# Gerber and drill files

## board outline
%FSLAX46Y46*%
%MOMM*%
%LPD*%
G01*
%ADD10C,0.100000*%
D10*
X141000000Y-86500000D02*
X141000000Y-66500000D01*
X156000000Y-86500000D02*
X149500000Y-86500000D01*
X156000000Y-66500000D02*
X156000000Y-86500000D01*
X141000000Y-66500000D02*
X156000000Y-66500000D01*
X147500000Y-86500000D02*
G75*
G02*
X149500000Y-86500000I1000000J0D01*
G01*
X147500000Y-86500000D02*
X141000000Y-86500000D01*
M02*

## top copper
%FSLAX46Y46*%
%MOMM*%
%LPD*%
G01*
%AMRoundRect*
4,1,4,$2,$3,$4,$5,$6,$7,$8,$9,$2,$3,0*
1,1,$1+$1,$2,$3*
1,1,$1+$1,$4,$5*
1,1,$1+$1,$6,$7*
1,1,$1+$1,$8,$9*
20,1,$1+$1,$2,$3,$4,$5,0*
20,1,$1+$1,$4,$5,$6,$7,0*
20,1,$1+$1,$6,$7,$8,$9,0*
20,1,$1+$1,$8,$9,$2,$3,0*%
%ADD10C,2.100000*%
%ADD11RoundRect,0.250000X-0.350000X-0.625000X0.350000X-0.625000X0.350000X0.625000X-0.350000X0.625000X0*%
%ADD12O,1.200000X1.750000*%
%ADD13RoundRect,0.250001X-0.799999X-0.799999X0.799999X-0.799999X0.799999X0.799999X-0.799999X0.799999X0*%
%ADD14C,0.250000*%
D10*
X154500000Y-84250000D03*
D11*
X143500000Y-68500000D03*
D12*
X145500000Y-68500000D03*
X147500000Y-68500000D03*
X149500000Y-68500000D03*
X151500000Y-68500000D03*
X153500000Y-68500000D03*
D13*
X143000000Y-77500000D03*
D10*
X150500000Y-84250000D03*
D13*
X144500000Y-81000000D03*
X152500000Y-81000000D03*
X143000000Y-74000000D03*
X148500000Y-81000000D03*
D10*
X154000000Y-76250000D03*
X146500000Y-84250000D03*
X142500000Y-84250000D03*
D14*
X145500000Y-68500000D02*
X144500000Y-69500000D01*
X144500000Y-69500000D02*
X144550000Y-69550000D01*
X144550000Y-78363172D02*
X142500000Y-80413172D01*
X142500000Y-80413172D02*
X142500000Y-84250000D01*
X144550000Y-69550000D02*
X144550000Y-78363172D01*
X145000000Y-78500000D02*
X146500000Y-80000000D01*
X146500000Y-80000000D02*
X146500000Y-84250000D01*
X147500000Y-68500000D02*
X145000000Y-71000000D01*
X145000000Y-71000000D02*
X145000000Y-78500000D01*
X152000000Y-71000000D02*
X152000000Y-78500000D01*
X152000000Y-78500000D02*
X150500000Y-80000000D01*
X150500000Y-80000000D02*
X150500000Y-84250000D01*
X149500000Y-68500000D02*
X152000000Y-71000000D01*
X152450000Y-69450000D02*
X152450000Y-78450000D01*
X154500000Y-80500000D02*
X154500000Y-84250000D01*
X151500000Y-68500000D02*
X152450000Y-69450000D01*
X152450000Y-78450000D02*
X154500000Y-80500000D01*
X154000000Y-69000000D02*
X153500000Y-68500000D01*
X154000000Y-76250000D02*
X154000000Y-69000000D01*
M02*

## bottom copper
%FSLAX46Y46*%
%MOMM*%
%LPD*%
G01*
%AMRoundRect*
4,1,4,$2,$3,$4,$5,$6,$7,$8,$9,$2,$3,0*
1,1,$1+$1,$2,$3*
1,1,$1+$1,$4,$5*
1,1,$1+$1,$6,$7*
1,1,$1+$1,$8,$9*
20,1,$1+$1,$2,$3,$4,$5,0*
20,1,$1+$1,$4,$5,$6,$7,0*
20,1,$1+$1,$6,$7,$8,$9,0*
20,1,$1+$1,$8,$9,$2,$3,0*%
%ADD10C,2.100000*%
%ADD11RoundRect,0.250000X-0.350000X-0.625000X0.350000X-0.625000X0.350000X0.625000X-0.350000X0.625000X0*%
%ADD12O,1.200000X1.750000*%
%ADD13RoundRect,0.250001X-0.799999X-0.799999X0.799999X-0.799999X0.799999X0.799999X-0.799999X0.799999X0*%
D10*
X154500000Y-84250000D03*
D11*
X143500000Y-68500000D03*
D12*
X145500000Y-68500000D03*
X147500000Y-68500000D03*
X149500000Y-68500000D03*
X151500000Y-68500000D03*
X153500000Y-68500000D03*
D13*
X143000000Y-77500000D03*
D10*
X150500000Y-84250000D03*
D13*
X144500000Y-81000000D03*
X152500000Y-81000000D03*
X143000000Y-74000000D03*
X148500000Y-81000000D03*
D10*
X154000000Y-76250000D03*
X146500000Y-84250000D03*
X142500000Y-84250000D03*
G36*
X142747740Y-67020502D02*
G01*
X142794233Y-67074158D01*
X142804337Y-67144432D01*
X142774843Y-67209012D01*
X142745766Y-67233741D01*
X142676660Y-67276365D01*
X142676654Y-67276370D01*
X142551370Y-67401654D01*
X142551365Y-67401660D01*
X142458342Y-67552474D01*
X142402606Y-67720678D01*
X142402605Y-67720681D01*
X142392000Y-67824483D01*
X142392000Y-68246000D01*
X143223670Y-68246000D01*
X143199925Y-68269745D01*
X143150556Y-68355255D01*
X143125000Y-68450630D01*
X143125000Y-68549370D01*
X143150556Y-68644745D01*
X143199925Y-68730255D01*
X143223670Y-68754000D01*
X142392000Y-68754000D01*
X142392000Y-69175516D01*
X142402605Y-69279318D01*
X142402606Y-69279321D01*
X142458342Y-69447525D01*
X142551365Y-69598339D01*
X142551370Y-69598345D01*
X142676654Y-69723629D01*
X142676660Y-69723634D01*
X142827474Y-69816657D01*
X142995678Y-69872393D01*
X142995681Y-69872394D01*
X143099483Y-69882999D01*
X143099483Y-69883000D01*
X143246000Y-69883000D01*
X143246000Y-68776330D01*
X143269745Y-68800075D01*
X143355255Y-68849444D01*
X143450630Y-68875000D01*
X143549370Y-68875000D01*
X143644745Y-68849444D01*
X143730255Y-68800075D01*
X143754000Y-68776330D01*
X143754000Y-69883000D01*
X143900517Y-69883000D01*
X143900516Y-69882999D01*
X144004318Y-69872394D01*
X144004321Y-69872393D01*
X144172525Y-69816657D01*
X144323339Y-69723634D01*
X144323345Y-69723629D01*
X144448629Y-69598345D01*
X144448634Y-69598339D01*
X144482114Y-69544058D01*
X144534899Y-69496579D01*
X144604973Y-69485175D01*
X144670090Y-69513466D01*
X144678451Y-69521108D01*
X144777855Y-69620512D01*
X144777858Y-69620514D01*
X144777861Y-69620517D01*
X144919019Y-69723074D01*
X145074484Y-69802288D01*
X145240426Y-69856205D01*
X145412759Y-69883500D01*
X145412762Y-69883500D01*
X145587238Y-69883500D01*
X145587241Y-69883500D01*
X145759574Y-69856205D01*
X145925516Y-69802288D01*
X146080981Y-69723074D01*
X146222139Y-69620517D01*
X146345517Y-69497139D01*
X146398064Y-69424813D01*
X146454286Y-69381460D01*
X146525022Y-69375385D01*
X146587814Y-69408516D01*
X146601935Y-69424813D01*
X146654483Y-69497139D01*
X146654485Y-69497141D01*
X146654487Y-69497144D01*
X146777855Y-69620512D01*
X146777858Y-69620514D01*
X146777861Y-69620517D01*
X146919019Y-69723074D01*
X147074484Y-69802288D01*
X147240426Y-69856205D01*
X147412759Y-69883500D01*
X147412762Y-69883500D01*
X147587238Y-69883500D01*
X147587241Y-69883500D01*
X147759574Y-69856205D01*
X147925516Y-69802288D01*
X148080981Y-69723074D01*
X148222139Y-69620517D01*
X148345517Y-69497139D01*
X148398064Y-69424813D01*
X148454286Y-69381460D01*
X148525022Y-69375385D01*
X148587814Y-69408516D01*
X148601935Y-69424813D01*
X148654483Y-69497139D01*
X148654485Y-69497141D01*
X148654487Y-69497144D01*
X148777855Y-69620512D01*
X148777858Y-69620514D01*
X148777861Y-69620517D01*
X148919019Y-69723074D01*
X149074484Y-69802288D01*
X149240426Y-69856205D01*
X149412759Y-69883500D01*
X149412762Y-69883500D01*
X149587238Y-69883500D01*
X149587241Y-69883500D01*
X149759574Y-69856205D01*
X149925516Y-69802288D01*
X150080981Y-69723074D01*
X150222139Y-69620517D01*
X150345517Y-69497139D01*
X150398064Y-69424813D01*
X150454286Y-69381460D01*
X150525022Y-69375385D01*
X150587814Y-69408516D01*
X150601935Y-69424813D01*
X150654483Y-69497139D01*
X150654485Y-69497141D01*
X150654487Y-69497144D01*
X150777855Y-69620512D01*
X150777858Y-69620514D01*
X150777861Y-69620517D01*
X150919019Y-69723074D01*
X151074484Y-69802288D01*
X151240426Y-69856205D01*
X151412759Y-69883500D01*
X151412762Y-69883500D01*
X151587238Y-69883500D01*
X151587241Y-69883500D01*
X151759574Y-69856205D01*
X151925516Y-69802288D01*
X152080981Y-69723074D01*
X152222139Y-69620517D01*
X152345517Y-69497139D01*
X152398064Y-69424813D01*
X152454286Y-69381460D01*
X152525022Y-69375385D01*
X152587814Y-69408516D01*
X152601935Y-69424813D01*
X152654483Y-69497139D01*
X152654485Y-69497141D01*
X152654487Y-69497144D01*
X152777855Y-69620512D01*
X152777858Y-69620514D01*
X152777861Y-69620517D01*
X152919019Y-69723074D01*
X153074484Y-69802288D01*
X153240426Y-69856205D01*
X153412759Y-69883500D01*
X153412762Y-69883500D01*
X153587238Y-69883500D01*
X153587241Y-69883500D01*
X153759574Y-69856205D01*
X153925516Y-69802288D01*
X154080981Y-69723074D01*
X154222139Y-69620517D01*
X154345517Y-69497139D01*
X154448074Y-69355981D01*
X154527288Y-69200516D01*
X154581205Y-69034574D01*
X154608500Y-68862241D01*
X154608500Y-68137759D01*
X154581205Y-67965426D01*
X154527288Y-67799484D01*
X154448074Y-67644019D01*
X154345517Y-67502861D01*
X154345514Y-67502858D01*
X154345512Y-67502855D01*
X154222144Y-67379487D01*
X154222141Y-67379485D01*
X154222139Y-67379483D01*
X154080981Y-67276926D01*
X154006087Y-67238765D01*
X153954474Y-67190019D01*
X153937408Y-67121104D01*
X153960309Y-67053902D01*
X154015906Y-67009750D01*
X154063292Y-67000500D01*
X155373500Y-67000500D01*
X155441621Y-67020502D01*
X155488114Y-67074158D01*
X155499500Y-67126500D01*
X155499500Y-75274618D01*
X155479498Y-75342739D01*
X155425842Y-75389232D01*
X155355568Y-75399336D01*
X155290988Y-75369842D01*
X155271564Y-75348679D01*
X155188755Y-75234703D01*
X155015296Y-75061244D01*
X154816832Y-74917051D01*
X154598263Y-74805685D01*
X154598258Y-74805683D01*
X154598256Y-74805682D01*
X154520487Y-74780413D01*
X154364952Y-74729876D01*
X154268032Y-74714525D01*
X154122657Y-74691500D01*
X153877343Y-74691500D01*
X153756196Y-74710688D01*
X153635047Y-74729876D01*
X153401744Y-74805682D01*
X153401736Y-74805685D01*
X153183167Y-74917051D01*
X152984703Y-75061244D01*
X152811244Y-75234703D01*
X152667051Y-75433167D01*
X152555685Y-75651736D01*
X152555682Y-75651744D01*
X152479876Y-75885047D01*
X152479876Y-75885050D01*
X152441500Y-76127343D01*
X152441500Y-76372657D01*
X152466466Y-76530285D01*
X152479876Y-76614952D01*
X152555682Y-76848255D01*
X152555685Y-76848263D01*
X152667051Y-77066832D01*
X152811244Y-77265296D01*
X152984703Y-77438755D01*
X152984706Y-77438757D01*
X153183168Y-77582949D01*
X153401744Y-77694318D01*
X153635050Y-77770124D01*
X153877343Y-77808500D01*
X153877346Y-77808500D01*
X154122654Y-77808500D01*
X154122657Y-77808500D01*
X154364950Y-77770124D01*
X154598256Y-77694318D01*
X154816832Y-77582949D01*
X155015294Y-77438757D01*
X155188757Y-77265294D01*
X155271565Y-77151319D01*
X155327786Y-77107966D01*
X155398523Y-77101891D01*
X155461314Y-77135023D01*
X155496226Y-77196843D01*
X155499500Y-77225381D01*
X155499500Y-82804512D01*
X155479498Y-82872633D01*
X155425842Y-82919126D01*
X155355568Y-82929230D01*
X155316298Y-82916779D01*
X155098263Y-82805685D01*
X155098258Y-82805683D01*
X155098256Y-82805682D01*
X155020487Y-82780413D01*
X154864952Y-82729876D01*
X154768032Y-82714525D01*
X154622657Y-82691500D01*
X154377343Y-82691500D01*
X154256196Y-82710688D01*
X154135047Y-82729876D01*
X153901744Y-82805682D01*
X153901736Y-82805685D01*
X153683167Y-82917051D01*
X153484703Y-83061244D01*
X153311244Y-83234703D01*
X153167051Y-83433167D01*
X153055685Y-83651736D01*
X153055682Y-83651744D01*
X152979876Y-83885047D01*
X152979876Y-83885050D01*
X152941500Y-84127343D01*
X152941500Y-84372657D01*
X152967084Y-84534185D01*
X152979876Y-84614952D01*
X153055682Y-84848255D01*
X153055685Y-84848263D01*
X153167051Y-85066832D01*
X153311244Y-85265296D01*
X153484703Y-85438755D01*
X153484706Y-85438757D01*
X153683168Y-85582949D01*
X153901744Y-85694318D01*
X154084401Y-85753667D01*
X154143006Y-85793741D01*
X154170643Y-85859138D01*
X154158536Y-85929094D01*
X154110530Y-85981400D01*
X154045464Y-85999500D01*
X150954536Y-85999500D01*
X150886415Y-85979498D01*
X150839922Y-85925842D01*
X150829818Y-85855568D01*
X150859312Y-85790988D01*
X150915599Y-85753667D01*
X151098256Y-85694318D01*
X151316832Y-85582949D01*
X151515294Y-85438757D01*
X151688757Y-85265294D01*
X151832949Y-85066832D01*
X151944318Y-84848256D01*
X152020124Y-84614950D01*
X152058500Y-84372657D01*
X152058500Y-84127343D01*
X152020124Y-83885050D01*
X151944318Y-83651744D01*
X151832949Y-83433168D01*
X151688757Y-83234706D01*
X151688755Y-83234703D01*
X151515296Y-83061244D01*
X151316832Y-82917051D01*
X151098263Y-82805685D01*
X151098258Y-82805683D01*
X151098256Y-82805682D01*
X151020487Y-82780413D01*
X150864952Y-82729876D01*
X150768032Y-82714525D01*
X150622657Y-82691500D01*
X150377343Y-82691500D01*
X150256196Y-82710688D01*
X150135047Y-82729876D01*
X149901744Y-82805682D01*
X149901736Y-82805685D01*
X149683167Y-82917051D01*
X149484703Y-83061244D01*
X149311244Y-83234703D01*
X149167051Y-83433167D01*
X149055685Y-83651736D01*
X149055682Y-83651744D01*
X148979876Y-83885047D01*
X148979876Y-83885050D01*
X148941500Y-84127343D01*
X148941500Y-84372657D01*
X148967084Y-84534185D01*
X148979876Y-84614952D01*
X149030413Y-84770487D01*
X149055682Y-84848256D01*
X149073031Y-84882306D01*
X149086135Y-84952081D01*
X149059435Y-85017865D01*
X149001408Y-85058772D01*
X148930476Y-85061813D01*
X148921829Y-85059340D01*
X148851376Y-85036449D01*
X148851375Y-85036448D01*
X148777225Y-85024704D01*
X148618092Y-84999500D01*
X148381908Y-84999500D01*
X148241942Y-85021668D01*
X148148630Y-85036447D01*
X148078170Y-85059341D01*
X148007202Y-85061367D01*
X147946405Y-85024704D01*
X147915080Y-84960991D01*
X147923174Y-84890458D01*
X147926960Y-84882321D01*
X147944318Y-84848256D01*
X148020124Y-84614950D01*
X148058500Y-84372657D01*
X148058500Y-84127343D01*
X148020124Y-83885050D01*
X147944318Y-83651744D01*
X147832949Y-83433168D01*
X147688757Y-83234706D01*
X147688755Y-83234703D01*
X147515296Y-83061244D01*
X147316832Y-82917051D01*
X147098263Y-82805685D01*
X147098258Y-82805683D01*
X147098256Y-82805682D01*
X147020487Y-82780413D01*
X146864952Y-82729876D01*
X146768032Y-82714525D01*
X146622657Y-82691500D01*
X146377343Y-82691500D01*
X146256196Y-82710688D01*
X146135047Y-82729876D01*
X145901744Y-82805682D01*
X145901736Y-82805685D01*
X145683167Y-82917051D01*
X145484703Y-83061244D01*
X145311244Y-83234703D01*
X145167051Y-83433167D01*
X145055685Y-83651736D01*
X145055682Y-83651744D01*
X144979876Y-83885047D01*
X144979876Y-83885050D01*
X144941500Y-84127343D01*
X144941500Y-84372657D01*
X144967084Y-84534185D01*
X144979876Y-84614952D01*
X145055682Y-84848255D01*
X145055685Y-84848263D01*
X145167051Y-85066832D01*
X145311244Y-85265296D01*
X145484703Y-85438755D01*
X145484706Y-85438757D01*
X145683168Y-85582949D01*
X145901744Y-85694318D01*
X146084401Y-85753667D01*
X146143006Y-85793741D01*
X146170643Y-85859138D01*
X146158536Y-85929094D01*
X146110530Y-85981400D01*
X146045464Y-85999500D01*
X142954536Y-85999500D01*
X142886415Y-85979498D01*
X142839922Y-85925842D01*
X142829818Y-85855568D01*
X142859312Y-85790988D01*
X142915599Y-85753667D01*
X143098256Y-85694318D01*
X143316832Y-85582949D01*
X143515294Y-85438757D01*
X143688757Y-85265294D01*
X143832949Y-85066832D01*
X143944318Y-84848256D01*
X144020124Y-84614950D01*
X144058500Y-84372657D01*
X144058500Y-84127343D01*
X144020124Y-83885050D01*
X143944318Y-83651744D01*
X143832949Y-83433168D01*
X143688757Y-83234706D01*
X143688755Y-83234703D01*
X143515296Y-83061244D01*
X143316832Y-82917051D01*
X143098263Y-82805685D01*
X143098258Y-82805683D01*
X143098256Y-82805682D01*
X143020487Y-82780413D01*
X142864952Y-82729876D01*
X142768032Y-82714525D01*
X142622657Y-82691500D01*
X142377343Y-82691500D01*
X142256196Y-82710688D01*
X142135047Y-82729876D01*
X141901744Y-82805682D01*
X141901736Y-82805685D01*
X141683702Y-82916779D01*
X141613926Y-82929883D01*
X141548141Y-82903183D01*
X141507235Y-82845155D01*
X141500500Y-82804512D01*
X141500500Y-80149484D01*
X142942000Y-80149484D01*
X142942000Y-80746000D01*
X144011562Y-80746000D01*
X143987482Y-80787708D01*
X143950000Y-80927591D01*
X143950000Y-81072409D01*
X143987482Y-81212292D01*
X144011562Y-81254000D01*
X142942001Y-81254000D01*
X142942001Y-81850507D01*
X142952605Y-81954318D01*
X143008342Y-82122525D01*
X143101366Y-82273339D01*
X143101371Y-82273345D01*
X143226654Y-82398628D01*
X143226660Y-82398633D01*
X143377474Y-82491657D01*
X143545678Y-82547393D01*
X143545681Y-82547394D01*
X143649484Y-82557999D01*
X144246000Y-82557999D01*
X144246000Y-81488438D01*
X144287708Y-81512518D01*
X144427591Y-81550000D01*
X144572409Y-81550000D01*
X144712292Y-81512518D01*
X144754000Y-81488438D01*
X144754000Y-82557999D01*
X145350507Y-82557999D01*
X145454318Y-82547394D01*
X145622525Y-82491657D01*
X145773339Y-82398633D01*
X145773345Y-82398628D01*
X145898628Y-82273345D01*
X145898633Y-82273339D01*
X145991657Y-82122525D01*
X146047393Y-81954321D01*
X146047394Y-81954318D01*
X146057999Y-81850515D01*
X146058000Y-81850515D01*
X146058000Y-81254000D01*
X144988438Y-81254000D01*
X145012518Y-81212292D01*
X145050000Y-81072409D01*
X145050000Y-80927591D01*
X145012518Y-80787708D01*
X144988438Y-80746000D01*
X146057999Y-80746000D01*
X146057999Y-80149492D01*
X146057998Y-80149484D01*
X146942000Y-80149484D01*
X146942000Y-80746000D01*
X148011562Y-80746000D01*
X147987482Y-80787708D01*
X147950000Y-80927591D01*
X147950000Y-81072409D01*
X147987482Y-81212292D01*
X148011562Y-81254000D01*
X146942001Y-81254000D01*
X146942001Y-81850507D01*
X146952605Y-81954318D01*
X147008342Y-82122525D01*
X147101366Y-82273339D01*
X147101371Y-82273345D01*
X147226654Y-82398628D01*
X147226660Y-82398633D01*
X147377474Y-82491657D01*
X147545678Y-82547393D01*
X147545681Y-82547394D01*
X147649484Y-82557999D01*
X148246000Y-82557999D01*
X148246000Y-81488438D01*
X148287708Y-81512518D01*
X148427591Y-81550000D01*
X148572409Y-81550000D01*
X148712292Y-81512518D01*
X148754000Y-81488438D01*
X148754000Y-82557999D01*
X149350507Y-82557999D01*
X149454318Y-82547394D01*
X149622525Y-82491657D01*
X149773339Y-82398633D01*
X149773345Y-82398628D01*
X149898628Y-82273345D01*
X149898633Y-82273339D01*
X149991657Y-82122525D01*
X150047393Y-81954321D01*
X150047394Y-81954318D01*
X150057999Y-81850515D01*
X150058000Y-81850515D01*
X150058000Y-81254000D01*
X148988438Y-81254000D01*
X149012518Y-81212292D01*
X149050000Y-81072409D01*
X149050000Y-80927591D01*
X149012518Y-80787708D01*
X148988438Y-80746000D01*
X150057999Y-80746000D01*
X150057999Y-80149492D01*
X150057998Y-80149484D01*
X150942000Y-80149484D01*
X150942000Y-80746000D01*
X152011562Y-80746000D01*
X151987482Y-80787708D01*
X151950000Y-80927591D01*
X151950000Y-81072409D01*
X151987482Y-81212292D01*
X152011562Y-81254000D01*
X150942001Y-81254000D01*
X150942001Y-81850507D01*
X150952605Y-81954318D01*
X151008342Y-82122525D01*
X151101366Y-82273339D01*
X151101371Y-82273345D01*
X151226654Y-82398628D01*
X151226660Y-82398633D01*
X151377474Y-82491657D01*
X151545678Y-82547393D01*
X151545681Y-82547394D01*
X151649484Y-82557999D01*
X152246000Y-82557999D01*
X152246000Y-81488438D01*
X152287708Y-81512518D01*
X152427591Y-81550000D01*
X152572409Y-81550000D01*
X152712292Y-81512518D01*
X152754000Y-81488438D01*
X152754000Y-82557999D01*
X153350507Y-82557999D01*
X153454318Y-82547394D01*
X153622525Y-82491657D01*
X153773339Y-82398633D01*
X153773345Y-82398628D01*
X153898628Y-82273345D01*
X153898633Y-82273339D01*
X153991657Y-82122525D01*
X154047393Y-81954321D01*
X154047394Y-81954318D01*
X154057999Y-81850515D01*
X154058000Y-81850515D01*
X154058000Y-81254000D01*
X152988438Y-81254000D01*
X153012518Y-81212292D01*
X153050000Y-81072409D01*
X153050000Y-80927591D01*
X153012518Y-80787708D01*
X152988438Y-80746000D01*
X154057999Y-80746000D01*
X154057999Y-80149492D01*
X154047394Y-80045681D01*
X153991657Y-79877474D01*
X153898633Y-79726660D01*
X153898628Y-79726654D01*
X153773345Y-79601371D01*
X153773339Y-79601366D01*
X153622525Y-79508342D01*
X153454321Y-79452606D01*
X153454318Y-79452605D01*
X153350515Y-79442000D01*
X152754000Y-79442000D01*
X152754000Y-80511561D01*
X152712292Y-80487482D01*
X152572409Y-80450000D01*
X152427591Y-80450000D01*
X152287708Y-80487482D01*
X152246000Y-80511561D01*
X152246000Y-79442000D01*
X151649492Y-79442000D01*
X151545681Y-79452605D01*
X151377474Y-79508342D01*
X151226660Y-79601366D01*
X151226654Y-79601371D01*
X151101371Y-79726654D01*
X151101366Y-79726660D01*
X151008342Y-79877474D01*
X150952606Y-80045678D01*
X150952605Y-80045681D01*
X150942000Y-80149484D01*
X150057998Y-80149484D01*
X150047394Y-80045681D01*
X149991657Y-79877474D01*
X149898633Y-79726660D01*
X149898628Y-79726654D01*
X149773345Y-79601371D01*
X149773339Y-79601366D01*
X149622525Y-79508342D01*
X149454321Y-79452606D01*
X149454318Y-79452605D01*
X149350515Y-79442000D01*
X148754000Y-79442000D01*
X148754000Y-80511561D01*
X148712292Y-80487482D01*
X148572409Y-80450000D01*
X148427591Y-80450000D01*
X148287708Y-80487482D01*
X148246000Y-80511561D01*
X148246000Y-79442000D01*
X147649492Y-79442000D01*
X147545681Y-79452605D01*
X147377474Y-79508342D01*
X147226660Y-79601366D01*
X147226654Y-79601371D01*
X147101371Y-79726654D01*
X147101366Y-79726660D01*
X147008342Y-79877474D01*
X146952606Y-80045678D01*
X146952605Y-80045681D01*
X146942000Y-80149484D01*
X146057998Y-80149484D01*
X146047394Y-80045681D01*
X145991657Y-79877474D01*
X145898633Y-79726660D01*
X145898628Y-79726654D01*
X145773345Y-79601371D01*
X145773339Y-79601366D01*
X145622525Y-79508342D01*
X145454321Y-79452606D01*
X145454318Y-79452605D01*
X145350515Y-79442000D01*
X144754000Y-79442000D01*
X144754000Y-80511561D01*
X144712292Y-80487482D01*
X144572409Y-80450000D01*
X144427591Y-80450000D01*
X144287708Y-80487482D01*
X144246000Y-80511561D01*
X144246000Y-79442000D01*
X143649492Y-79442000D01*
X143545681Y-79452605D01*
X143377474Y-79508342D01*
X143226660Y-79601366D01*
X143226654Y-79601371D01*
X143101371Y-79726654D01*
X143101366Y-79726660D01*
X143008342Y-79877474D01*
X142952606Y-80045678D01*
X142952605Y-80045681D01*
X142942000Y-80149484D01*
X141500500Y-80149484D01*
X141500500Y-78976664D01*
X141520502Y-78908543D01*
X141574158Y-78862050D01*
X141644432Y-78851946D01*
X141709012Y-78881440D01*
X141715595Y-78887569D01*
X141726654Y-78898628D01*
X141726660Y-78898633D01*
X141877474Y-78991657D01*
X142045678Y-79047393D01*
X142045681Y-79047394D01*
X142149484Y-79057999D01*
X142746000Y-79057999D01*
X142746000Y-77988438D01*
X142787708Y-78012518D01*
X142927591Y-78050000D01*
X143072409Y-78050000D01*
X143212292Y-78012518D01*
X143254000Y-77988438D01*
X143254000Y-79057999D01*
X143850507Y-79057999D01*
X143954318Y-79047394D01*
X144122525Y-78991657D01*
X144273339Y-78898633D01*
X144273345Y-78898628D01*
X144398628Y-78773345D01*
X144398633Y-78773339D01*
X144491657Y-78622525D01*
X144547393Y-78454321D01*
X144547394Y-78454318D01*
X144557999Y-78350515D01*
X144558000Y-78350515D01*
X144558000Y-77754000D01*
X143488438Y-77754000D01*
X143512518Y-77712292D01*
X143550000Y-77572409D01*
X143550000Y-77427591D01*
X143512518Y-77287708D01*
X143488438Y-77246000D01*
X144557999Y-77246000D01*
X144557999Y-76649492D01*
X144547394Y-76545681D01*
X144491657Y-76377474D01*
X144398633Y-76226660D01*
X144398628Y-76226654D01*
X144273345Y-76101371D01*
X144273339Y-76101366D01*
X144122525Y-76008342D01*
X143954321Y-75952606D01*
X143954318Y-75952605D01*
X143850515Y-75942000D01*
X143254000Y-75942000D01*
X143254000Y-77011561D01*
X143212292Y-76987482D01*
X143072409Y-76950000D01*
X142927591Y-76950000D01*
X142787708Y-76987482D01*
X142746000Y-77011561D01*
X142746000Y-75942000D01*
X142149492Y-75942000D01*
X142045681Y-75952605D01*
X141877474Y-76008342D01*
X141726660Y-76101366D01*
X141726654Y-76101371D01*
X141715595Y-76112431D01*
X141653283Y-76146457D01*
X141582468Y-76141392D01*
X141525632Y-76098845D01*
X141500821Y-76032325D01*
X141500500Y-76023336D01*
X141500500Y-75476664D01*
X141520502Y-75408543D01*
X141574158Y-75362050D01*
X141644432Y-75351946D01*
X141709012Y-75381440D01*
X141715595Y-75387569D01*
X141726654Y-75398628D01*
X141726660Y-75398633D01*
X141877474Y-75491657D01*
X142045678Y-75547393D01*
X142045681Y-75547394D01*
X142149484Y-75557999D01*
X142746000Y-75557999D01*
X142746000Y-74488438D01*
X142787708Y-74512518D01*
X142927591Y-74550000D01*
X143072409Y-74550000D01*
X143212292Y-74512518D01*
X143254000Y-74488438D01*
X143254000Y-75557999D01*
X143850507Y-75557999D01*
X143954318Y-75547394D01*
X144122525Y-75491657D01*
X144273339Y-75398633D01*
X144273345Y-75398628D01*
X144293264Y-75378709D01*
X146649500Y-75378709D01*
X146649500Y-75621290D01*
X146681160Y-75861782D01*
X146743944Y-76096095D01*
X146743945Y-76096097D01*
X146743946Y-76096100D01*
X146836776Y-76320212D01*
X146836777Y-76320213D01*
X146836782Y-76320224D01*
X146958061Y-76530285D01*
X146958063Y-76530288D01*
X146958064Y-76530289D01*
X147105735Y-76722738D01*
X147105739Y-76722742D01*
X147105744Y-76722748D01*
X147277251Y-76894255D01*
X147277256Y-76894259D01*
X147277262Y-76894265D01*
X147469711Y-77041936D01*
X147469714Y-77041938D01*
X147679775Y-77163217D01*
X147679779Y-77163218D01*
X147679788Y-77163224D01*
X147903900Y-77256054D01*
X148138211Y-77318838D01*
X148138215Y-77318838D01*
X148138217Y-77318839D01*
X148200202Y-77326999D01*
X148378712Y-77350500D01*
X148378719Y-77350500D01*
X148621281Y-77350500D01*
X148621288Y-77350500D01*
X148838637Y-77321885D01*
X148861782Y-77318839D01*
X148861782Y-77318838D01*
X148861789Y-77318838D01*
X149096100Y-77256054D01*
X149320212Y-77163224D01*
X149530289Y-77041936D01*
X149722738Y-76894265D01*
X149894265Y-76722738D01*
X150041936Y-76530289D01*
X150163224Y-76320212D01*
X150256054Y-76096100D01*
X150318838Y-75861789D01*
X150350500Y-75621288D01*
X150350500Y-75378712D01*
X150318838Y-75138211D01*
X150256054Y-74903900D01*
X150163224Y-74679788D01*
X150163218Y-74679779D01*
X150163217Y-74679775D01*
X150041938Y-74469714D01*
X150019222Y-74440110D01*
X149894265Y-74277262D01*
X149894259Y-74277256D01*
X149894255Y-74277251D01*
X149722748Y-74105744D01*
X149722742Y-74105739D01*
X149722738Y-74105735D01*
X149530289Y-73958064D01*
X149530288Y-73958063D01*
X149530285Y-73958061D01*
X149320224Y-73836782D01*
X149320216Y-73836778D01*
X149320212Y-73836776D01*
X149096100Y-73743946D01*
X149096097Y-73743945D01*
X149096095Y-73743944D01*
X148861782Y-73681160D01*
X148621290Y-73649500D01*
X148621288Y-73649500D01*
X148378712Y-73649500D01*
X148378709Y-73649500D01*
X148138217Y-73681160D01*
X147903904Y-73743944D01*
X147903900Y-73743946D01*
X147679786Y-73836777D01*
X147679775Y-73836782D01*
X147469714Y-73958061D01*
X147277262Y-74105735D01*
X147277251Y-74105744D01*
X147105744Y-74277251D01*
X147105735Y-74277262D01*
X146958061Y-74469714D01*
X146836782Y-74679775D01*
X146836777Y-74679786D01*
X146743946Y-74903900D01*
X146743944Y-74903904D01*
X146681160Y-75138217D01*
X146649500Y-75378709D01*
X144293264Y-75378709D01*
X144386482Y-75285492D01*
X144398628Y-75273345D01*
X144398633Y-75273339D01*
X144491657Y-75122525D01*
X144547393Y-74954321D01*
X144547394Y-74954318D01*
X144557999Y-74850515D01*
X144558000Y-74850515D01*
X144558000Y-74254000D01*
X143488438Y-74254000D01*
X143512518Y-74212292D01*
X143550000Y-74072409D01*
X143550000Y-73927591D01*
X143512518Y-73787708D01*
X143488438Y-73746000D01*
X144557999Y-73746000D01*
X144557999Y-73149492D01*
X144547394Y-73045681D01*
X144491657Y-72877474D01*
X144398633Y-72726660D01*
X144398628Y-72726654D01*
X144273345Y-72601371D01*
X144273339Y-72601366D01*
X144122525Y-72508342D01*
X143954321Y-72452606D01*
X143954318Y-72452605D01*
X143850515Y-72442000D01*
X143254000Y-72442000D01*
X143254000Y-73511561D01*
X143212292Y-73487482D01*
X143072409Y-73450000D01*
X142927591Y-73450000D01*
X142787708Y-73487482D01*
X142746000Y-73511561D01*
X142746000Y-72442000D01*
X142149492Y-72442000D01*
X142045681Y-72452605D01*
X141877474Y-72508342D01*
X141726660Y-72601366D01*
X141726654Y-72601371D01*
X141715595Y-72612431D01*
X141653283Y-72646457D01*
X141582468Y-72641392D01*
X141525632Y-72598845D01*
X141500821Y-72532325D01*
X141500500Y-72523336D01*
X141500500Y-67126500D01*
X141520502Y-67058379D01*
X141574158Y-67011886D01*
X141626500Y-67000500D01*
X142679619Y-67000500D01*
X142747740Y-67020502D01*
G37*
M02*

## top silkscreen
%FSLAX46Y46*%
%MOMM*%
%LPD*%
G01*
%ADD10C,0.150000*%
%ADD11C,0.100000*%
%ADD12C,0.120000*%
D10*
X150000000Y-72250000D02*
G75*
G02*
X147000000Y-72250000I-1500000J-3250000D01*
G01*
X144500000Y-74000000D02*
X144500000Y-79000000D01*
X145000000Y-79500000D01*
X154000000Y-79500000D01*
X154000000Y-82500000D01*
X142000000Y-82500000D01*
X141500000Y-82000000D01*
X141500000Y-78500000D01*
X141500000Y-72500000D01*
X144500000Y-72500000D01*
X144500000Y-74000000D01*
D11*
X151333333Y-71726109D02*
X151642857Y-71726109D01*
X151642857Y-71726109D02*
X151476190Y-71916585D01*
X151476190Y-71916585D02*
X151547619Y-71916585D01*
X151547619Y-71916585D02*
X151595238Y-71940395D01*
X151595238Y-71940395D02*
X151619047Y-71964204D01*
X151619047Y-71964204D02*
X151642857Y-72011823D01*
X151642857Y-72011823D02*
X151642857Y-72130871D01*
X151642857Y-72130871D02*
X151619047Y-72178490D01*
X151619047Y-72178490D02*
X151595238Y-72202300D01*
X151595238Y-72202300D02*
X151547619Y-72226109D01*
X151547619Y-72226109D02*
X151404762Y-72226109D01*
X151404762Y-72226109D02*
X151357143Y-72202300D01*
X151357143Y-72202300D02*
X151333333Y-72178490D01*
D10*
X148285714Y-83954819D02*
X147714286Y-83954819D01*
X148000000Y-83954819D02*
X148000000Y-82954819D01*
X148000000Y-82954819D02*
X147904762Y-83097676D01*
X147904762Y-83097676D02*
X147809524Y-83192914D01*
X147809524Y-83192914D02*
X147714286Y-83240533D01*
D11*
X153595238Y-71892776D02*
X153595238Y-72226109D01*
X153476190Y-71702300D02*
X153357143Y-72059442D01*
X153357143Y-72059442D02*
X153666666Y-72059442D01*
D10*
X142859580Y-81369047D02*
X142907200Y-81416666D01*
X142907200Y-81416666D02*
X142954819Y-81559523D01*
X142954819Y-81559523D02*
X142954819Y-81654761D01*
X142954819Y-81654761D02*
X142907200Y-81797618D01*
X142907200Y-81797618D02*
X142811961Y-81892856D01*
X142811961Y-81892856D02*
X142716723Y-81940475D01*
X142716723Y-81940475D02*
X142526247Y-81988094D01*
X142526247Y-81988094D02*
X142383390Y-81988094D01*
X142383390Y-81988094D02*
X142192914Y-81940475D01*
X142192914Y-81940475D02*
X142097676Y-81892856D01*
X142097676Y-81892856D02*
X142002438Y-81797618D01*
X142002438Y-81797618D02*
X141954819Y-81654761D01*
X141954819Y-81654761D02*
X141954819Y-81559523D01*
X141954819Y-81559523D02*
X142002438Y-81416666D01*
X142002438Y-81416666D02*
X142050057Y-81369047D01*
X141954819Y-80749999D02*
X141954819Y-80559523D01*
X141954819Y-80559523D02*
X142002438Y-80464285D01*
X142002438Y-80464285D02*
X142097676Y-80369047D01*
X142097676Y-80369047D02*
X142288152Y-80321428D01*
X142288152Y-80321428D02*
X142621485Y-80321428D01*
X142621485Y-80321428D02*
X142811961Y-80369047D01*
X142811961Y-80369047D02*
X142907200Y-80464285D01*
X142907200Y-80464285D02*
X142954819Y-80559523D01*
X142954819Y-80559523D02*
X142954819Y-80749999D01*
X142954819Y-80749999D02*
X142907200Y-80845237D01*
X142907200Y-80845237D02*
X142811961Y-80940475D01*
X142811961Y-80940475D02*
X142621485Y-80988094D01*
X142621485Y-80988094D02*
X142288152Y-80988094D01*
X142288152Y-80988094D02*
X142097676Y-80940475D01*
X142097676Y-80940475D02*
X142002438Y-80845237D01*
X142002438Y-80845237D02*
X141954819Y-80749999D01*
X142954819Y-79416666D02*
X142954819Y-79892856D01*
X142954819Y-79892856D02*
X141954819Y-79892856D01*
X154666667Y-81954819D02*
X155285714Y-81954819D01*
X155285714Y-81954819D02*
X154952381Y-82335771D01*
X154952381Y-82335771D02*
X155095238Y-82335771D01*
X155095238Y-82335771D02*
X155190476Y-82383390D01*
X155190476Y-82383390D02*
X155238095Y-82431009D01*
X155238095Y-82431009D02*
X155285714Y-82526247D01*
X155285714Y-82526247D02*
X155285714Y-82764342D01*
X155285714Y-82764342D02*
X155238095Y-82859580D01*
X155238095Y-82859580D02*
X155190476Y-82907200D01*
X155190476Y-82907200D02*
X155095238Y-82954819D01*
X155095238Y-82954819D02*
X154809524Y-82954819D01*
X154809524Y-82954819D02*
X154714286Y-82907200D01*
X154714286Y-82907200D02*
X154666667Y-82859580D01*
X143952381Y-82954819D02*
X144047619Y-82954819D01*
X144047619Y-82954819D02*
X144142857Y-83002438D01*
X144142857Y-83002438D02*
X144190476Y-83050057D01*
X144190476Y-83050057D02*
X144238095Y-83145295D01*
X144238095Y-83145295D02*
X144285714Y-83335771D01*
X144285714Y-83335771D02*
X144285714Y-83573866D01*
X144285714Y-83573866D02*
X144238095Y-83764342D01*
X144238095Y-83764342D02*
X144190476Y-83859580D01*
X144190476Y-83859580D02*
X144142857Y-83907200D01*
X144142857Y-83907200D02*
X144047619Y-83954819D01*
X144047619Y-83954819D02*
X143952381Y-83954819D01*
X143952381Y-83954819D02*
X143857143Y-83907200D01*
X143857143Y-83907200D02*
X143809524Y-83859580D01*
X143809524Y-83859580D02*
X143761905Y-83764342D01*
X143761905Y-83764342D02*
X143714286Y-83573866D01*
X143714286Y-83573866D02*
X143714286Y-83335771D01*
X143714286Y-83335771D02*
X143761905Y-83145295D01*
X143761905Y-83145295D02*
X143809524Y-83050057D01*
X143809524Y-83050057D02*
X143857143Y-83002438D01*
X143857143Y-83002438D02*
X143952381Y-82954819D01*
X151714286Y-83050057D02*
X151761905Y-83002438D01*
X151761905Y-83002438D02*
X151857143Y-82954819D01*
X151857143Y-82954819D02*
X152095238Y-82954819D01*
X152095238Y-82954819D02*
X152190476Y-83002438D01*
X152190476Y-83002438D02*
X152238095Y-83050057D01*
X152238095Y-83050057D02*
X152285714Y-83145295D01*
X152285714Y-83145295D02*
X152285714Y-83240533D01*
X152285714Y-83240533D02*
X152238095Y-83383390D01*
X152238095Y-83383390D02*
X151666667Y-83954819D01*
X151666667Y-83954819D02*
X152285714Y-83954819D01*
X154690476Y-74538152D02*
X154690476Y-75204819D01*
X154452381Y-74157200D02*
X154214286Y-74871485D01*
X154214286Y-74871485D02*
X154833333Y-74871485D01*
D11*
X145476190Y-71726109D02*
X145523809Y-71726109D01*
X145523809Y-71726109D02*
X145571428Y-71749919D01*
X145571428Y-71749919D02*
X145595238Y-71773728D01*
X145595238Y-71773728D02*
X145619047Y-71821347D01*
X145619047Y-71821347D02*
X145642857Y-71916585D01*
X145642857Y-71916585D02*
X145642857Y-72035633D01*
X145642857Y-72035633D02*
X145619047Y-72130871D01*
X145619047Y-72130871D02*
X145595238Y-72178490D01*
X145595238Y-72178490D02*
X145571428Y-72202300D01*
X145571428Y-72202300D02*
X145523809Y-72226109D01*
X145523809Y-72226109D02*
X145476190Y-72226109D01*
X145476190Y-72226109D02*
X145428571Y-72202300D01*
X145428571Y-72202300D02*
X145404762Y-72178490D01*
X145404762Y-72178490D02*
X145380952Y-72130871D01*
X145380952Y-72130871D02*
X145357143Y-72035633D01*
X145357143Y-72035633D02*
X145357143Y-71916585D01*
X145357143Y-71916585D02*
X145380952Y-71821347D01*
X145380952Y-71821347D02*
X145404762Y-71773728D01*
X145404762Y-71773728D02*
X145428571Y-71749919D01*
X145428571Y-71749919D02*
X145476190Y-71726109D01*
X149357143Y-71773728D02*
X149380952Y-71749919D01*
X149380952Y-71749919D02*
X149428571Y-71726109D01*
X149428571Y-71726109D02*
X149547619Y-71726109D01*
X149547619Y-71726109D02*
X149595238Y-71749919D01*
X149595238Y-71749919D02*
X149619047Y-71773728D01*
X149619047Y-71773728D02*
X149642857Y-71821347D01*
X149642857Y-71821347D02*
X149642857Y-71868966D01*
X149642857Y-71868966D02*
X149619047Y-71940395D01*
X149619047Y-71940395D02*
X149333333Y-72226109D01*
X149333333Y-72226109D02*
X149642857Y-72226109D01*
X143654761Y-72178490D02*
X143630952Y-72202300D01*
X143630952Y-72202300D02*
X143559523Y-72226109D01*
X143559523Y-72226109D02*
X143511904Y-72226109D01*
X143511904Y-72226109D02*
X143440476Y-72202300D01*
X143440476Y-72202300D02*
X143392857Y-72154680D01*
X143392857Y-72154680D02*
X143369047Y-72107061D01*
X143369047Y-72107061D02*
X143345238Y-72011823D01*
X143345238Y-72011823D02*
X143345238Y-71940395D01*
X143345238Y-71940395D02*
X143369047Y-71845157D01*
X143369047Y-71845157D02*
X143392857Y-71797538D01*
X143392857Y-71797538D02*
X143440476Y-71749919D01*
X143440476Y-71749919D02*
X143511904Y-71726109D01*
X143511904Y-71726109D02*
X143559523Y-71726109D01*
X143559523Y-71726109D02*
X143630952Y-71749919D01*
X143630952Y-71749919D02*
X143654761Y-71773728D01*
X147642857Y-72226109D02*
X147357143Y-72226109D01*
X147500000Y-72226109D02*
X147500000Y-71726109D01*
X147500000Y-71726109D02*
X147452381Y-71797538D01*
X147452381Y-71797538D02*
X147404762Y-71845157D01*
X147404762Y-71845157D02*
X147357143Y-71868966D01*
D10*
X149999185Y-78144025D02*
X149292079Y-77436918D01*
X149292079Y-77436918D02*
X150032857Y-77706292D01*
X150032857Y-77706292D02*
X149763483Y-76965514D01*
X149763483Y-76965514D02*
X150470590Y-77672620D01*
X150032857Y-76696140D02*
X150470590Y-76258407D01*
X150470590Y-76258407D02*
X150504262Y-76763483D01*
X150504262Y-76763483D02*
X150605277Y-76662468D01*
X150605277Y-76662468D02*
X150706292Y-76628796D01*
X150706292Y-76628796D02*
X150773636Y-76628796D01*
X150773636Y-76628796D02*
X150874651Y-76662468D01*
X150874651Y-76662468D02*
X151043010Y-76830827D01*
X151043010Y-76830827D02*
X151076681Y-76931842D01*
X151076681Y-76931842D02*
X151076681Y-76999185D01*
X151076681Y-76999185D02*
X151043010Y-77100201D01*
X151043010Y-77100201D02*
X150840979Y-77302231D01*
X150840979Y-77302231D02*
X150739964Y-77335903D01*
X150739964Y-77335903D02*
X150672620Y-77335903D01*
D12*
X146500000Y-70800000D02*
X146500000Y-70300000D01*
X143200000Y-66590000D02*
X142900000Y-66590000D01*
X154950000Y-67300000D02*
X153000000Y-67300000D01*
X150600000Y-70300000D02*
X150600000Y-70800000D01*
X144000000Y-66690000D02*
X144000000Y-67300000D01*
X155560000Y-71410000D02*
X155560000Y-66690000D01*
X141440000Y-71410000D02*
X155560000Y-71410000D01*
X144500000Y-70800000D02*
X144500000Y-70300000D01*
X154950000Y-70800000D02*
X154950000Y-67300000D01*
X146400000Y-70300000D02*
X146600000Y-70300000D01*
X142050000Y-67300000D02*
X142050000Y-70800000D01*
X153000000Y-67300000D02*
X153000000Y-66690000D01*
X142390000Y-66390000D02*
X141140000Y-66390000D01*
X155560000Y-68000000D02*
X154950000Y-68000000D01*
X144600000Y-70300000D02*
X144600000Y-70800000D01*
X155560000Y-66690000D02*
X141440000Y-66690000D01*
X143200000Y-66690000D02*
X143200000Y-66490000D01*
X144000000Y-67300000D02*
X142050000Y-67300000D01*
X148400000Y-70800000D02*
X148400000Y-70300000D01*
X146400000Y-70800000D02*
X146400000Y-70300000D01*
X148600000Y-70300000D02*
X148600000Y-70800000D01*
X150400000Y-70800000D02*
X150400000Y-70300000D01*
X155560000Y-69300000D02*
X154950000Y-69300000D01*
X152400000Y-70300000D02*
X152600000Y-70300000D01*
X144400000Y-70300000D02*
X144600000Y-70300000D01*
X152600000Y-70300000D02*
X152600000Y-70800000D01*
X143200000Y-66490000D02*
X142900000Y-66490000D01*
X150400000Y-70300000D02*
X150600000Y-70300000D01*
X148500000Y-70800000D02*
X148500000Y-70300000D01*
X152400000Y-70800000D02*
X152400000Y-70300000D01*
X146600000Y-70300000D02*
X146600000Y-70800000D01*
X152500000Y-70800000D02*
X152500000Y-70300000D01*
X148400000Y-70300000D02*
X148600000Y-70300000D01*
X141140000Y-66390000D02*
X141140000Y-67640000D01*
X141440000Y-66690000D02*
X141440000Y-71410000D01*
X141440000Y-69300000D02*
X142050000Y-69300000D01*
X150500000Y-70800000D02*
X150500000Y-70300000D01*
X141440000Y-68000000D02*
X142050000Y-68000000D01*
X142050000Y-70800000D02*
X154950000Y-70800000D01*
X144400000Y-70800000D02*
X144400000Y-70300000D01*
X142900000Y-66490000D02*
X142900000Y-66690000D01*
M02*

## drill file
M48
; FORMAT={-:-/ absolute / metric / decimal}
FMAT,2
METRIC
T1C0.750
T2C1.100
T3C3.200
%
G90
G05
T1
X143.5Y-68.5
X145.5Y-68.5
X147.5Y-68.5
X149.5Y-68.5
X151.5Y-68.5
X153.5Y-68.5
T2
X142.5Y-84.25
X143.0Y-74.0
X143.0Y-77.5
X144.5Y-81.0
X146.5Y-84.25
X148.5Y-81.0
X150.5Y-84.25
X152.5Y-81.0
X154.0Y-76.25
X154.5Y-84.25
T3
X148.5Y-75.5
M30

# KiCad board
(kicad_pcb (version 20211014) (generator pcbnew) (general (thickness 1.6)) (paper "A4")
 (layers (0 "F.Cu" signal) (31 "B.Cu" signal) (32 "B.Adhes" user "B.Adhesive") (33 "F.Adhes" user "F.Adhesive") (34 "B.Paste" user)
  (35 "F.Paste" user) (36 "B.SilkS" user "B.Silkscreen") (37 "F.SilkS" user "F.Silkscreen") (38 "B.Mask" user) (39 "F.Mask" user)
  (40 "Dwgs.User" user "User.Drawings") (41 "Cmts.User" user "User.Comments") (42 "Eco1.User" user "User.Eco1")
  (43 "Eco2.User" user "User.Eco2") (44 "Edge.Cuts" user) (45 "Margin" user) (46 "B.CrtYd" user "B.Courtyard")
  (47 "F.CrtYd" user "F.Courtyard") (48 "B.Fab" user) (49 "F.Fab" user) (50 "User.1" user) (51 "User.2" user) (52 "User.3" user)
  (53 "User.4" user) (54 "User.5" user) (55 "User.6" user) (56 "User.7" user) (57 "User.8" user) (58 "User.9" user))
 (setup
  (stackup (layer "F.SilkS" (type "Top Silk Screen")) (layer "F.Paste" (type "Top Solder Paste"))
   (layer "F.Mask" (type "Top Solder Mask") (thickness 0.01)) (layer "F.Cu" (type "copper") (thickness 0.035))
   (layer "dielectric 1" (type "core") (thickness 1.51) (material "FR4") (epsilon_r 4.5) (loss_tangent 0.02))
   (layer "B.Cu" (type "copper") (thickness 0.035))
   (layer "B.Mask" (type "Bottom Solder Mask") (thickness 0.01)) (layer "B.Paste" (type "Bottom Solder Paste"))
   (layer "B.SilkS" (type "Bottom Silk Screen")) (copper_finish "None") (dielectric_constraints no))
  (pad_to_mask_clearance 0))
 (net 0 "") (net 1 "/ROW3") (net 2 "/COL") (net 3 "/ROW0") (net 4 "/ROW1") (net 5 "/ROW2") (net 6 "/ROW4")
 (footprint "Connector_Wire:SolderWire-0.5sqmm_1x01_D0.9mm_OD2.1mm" (layer "F.Cu") (at 154.5 84.25)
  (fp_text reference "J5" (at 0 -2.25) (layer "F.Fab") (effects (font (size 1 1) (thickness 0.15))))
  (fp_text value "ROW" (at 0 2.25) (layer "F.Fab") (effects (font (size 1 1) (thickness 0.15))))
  (pad "1" thru_hole circle (at 0 0) (size 2.1 2.1) (drill 1.1) (layers *.Cu *.Mask) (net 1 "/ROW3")))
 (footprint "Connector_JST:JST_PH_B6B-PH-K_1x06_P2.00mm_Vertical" (layer "F.Cu") (at 143.5 68.5)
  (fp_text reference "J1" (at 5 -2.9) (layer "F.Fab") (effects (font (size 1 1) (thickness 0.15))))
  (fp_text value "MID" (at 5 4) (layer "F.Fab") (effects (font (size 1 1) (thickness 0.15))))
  (fp_line (start 3 2.3) (end 3 1.8) (layer "F.SilkS") (width 0.12))
  (fp_line (start -0.3 -1.91) (end -0.6 -1.91) (layer "F.SilkS") (width 0.12))
  (fp_line (start 11.45 -1.2) (end 9.5 -1.2) (layer "F.SilkS") (width 0.12))
  (fp_line (start 7.1 1.8) (end 7.1 2.3) (layer "F.SilkS") (width 0.12))
  (fp_line (start 0.5 -1.81) (end 0.5 -1.2) (layer "F.SilkS") (width 0.12))
  (fp_line (start 12.06 2.91) (end 12.06 -1.81) (layer "F.SilkS") (width 0.12))
  (fp_line (start -2.06 2.91) (end 12.06 2.91) (layer "F.SilkS") (width 0.12))
  (fp_line (start 1 2.3) (end 1 1.8) (layer "F.SilkS") (width 0.12))
  (fp_line (start 11.45 2.3) (end 11.45 -1.2) (layer "F.SilkS") (width 0.12))
  (fp_line (start 2.9 1.8) (end 3.1 1.8) (layer "F.SilkS") (width 0.12))
  (fp_line (start -1.45 -1.2) (end -1.45 2.3) (layer "F.SilkS") (width 0.12))
  (fp_line (start 9.5 -1.2) (end 9.5 -1.81) (layer "F.SilkS") (width 0.12))
  (fp_line (start -1.11 -2.11) (end -2.36 -2.11) (layer "F.SilkS") (width 0.12))
  (fp_line (start 12.06 -0.5) (end 11.45 -0.5) (layer "F.SilkS") (width 0.12))
  (fp_line (start 1.1 1.8) (end 1.1 2.3) (layer "F.SilkS") (width 0.12))
  (fp_line (start 12.06 -1.81) (end -2.06 -1.81) (layer "F.SilkS") (width 0.12))
  (fp_line (start -0.3 -1.81) (end -0.3 -2.01) (layer "F.SilkS") (width 0.12))
  (fp_line (start 0.5 -1.2) (end -1.45 -1.2) (layer "F.SilkS") (width 0.12))
  (fp_line (start 4.9 2.3) (end 4.9 1.8) (layer "F.SilkS") (width 0.12))
  (fp_line (start 2.9 2.3) (end 2.9 1.8) (layer "F.SilkS") (width 0.12))
  (fp_line (start 5.1 1.8) (end 5.1 2.3) (layer "F.SilkS") (width 0.12))
  (fp_line (start 6.9 2.3) (end 6.9 1.8) (layer "F.SilkS") (width 0.12))
  (fp_line (start 12.06 0.8) (end 11.45 0.8) (layer "F.SilkS") (width 0.12))
  (fp_line (start 8.9 1.8) (end 9.1 1.8) (layer "F.SilkS") (width 0.12))
  (fp_line (start 0.9 1.8) (end 1.1 1.8) (layer "F.SilkS") (width 0.12))
  (fp_line (start 9.1 1.8) (end 9.1 2.3) (layer "F.SilkS") (width 0.12))
  (fp_line (start -0.3 -2.01) (end -0.6 -2.01) (layer "F.SilkS") (width 0.12))
  (fp_line (start 6.9 1.8) (end 7.1 1.8) (layer "F.SilkS") (width 0.12))
  (fp_line (start 5 2.3) (end 5 1.8) (layer "F.SilkS") (width 0.12))
  (fp_line (start 8.9 2.3) (end 8.9 1.8) (layer "F.SilkS") (width 0.12))
  (fp_line (start 3.1 1.8) (end 3.1 2.3) (layer "F.SilkS") (width 0.12))
  (fp_line (start 9 2.3) (end 9 1.8) (layer "F.SilkS") (width 0.12))
  (fp_line (start 4.9 1.8) (end 5.1 1.8) (layer "F.SilkS") (width 0.12))
  (fp_line (start -2.36 -2.11) (end -2.36 -0.86) (layer "F.SilkS") (width 0.12))
  (fp_line (start -2.06 -1.81) (end -2.06 2.91) (layer "F.SilkS") (width 0.12))
  (fp_line (start -2.06 0.8) (end -1.45 0.8) (layer "F.SilkS") (width 0.12))
  (fp_line (start 7 2.3) (end 7 1.8) (layer "F.SilkS") (width 0.12))
  (fp_line (start -2.06 -0.5) (end -1.45 -0.5) (layer "F.SilkS") (width 0.12))
  (fp_line (start -1.45 2.3) (end 11.45 2.3) (layer "F.SilkS") (width 0.12))
  (fp_line (start 0.9 2.3) (end 0.9 1.8) (layer "F.SilkS") (width 0.12))
  (fp_line (start -0.6 -2.01) (end -0.6 -1.81) (layer "F.SilkS") (width 0.12))
  (pad "1" thru_hole roundrect (at 0 0) (size 1.2 1.75) (drill 0.75) (layers *.Cu *.Mask) (roundrect_rratio 0.208333) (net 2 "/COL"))
  (pad "2" thru_hole oval (at 2 0) (size 1.2 1.75) (drill 0.75) (layers *.Cu *.Mask) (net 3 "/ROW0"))
  (pad "3" thru_hole oval (at 4 0) (size 1.2 1.75) (drill 0.75) (layers *.Cu *.Mask) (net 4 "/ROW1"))
  (pad "4" thru_hole oval (at 6 0) (size 1.2 1.75) (drill 0.75) (layers *.Cu *.Mask) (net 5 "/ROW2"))
  (pad "5" thru_hole oval (at 8 0) (size 1.2 1.75) (drill 0.75) (layers *.Cu *.Mask) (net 1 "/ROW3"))
  (pad "6" thru_hole oval (at 10 0) (size 1.2 1.75) (drill 0.75) (layers *.Cu *.Mask) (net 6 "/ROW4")))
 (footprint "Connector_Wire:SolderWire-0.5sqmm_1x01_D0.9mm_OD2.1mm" (layer "F.Cu") (at 143 77.5)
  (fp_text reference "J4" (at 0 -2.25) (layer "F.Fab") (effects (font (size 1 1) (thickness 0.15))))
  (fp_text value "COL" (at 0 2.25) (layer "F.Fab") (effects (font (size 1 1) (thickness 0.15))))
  (pad "1" thru_hole roundrect (at 0 0) (size 2.1 2.1) (drill 1.1) (layers *.Cu *.Mask) (roundrect_rratio 0.119048) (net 2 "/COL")))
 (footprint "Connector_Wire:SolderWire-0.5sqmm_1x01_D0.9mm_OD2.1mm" (layer "F.Cu") (at 150.5 84.25)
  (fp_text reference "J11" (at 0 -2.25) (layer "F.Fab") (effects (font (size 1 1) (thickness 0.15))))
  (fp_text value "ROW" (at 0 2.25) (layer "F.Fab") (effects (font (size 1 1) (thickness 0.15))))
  (pad "1" thru_hole circle (at 0 0) (size 2.1 2.1) (drill 1.1) (layers *.Cu *.Mask) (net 5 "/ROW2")))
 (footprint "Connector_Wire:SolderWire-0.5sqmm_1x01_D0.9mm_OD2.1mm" (layer "F.Cu") (at 144.5 81)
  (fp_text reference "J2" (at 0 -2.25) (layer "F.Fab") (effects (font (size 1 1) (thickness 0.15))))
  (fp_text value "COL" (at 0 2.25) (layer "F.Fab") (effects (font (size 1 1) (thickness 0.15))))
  (pad "1" thru_hole roundrect (at 0 0) (size 2.1 2.1) (drill 1.1) (layers *.Cu *.Mask) (roundrect_rratio 0.119048) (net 2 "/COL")))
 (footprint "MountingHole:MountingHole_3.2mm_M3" (layer "F.Cu") (at 148.5 75.5)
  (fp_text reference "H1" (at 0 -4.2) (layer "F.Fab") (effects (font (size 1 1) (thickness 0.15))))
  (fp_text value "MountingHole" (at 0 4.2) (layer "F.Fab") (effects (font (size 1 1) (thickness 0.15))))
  (pad "" np_thru_hole circle (at 0 0) (size 3.2 3.2) (drill 3.2) (layers *.Cu *.Mask)))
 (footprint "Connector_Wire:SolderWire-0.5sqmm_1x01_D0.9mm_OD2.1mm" (layer "F.Cu") (at 152.5 81)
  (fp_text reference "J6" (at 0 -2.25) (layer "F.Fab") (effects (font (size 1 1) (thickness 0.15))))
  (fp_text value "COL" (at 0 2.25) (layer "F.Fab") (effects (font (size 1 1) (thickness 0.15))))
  (pad "1" thru_hole roundrect (at 0 0) (size 2.1 2.1) (drill 1.1) (layers *.Cu *.Mask) (roundrect_rratio 0.119048) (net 2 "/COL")))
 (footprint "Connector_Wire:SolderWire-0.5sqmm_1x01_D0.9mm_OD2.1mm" (layer "F.Cu") (at 143 74)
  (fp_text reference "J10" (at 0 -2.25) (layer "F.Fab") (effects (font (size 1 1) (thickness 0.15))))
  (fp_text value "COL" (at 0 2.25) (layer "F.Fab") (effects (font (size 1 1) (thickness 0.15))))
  (pad "1" thru_hole roundrect (at 0 0) (size 2.1 2.1) (drill 1.1) (layers *.Cu *.Mask) (roundrect_rratio 0.119048) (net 2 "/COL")))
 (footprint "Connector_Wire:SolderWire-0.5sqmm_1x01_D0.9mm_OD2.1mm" (layer "F.Cu") (at 148.5 81)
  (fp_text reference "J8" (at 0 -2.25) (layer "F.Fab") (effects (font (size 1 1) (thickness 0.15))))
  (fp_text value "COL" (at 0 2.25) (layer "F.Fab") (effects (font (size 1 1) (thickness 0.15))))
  (pad "1" thru_hole roundrect (at 0 0) (size 2.1 2.1) (drill 1.1) (layers *.Cu *.Mask) (roundrect_rratio 0.119048) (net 2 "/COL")))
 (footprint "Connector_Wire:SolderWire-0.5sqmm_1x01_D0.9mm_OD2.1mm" (layer "F.Cu") (at 154 76.25)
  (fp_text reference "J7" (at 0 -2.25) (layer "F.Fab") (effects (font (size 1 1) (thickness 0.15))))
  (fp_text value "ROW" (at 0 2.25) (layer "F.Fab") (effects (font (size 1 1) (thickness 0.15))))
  (pad "1" thru_hole circle (at 0 0) (size 2.1 2.1) (drill 1.1) (layers *.Cu *.Mask) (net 6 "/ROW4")))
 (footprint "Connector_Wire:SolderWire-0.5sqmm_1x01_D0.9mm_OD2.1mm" (layer "F.Cu") (at 146.5 84.25)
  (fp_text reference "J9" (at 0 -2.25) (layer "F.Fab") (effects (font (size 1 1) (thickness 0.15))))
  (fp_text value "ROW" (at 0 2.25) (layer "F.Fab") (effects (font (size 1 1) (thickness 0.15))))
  (pad "1" thru_hole circle (at 0 0) (size 2.1 2.1) (drill 1.1) (layers *.Cu *.Mask) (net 4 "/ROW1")))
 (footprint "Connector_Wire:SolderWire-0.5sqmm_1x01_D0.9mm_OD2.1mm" (layer "F.Cu") (at 142.5 84.25)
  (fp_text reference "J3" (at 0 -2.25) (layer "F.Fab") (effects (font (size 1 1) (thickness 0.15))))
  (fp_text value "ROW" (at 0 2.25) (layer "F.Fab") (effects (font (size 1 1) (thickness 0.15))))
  (pad "1" thru_hole circle (at 0 0) (size 2.1 2.1) (drill 1.1) (layers *.Cu *.Mask) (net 3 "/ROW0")))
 (gr_arc (start 150 72.25) (mid 148.5 79.079455) (end 147 72.25) (layer "F.SilkS") (width 0.15))
 (gr_poly
  (pts (xy 144.5 74) (xy 144.5 79) (xy 145 79.5) (xy 154 79.5) (xy 154 82.5) (xy 142 82.5) (xy 141.5 82) (xy 141.5 78.5) (xy 141.5 72.5)
   (xy 144.5 72.5))
  (layer "F.SilkS") (width 0.15) (fill none))
 (gr_line (start 141 86.5) (end 141 66.5) (layer "Edge.Cuts") (width 0.1))
 (gr_line (start 156 86.5) (end 149.5 86.5) (layer "Edge.Cuts") (width 0.1))
 (gr_line (start 156 66.5) (end 156 86.5) (layer "Edge.Cuts") (width 0.1))
 (gr_line (start 141 66.5) (end 156 66.5) (layer "Edge.Cuts") (width 0.1))
 (gr_arc (start 147.5 86.5) (mid 148.5 85.5) (end 149.5 86.5) (layer "Edge.Cuts") (width 0.1))
 (gr_line (start 147.5 86.5) (end 141 86.5) (layer "Edge.Cuts") (width 0.1))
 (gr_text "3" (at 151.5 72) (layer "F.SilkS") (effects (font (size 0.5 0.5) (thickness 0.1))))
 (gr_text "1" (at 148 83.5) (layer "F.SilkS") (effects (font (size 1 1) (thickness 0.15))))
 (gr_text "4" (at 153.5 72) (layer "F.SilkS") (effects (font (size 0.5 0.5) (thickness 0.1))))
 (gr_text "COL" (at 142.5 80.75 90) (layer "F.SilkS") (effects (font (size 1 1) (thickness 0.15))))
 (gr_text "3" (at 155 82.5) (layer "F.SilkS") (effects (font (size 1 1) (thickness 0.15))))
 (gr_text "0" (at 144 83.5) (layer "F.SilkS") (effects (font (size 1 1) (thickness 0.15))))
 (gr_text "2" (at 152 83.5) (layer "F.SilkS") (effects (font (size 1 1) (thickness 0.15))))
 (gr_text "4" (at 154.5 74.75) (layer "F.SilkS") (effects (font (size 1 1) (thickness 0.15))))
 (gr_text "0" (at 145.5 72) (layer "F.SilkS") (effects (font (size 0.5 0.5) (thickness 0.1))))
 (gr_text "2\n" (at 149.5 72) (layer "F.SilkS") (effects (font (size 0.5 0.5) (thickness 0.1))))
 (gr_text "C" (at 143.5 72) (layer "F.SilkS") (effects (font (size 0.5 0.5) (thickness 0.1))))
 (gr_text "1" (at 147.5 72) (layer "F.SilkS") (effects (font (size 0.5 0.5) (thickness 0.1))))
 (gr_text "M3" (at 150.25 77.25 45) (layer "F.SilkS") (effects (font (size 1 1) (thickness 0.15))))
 (segment (start 145.5 68.5) (end 144.5 69.5) (width 0.25) (layer "F.Cu") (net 3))
 (segment (start 144.5 69.5) (end 144.55 69.55) (width 0.25) (layer "F.Cu") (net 3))
 (segment (start 144.55 78.363172) (end 142.5 80.413172) (width 0.25) (layer "F.Cu") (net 3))
 (segment (start 142.5 80.413172) (end 142.5 84.25) (width 0.25) (layer "F.Cu") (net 3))
 (segment (start 144.55 69.55) (end 144.55 78.363172) (width 0.25) (layer "F.Cu") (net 3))
 (segment (start 145 78.5) (end 146.5 80) (width 0.25) (layer "F.Cu") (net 4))
 (segment (start 146.5 80) (end 146.5 84.25) (width 0.25) (layer "F.Cu") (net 4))
 (segment (start 147.5 68.5) (end 145 71) (width 0.25) (layer "F.Cu") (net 4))
 (segment (start 145 71) (end 145 78.5) (width 0.25) (layer "F.Cu") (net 4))
 (segment (start 152 71) (end 152 78.5) (width 0.25) (layer "F.Cu") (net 5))
 (segment (start 152 78.5) (end 150.5 80) (width 0.25) (layer "F.Cu") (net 5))
 (segment (start 150.5 80) (end 150.5 84.25) (width 0.25) (layer "F.Cu") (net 5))
 (segment (start 149.5 68.5) (end 152 71) (width 0.25) (layer "F.Cu") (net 5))
 (segment (start 152.45 69.45) (end 152.45 78.45) (width 0.25) (layer "F.Cu") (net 1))
 (segment (start 154.5 80.5) (end 154.5 84.25) (width 0.25) (layer "F.Cu") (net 1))
 (segment (start 151.5 68.5) (end 152.45 69.45) (width 0.25) (layer "F.Cu") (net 1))
 (segment (start 152.45 78.45) (end 154.5 80.5) (width 0.25) (layer "F.Cu") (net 1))
 (segment (start 154 69) (end 153.5 68.5) (width 0.25) (layer "F.Cu") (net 6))
 (segment (start 154 76.25) (end 154 69) (width 0.25) (layer "F.Cu") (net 6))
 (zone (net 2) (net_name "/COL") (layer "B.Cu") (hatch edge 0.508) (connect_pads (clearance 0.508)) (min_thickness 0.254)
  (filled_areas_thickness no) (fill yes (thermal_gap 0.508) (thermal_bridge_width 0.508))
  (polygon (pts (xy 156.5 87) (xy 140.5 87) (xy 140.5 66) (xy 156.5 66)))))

